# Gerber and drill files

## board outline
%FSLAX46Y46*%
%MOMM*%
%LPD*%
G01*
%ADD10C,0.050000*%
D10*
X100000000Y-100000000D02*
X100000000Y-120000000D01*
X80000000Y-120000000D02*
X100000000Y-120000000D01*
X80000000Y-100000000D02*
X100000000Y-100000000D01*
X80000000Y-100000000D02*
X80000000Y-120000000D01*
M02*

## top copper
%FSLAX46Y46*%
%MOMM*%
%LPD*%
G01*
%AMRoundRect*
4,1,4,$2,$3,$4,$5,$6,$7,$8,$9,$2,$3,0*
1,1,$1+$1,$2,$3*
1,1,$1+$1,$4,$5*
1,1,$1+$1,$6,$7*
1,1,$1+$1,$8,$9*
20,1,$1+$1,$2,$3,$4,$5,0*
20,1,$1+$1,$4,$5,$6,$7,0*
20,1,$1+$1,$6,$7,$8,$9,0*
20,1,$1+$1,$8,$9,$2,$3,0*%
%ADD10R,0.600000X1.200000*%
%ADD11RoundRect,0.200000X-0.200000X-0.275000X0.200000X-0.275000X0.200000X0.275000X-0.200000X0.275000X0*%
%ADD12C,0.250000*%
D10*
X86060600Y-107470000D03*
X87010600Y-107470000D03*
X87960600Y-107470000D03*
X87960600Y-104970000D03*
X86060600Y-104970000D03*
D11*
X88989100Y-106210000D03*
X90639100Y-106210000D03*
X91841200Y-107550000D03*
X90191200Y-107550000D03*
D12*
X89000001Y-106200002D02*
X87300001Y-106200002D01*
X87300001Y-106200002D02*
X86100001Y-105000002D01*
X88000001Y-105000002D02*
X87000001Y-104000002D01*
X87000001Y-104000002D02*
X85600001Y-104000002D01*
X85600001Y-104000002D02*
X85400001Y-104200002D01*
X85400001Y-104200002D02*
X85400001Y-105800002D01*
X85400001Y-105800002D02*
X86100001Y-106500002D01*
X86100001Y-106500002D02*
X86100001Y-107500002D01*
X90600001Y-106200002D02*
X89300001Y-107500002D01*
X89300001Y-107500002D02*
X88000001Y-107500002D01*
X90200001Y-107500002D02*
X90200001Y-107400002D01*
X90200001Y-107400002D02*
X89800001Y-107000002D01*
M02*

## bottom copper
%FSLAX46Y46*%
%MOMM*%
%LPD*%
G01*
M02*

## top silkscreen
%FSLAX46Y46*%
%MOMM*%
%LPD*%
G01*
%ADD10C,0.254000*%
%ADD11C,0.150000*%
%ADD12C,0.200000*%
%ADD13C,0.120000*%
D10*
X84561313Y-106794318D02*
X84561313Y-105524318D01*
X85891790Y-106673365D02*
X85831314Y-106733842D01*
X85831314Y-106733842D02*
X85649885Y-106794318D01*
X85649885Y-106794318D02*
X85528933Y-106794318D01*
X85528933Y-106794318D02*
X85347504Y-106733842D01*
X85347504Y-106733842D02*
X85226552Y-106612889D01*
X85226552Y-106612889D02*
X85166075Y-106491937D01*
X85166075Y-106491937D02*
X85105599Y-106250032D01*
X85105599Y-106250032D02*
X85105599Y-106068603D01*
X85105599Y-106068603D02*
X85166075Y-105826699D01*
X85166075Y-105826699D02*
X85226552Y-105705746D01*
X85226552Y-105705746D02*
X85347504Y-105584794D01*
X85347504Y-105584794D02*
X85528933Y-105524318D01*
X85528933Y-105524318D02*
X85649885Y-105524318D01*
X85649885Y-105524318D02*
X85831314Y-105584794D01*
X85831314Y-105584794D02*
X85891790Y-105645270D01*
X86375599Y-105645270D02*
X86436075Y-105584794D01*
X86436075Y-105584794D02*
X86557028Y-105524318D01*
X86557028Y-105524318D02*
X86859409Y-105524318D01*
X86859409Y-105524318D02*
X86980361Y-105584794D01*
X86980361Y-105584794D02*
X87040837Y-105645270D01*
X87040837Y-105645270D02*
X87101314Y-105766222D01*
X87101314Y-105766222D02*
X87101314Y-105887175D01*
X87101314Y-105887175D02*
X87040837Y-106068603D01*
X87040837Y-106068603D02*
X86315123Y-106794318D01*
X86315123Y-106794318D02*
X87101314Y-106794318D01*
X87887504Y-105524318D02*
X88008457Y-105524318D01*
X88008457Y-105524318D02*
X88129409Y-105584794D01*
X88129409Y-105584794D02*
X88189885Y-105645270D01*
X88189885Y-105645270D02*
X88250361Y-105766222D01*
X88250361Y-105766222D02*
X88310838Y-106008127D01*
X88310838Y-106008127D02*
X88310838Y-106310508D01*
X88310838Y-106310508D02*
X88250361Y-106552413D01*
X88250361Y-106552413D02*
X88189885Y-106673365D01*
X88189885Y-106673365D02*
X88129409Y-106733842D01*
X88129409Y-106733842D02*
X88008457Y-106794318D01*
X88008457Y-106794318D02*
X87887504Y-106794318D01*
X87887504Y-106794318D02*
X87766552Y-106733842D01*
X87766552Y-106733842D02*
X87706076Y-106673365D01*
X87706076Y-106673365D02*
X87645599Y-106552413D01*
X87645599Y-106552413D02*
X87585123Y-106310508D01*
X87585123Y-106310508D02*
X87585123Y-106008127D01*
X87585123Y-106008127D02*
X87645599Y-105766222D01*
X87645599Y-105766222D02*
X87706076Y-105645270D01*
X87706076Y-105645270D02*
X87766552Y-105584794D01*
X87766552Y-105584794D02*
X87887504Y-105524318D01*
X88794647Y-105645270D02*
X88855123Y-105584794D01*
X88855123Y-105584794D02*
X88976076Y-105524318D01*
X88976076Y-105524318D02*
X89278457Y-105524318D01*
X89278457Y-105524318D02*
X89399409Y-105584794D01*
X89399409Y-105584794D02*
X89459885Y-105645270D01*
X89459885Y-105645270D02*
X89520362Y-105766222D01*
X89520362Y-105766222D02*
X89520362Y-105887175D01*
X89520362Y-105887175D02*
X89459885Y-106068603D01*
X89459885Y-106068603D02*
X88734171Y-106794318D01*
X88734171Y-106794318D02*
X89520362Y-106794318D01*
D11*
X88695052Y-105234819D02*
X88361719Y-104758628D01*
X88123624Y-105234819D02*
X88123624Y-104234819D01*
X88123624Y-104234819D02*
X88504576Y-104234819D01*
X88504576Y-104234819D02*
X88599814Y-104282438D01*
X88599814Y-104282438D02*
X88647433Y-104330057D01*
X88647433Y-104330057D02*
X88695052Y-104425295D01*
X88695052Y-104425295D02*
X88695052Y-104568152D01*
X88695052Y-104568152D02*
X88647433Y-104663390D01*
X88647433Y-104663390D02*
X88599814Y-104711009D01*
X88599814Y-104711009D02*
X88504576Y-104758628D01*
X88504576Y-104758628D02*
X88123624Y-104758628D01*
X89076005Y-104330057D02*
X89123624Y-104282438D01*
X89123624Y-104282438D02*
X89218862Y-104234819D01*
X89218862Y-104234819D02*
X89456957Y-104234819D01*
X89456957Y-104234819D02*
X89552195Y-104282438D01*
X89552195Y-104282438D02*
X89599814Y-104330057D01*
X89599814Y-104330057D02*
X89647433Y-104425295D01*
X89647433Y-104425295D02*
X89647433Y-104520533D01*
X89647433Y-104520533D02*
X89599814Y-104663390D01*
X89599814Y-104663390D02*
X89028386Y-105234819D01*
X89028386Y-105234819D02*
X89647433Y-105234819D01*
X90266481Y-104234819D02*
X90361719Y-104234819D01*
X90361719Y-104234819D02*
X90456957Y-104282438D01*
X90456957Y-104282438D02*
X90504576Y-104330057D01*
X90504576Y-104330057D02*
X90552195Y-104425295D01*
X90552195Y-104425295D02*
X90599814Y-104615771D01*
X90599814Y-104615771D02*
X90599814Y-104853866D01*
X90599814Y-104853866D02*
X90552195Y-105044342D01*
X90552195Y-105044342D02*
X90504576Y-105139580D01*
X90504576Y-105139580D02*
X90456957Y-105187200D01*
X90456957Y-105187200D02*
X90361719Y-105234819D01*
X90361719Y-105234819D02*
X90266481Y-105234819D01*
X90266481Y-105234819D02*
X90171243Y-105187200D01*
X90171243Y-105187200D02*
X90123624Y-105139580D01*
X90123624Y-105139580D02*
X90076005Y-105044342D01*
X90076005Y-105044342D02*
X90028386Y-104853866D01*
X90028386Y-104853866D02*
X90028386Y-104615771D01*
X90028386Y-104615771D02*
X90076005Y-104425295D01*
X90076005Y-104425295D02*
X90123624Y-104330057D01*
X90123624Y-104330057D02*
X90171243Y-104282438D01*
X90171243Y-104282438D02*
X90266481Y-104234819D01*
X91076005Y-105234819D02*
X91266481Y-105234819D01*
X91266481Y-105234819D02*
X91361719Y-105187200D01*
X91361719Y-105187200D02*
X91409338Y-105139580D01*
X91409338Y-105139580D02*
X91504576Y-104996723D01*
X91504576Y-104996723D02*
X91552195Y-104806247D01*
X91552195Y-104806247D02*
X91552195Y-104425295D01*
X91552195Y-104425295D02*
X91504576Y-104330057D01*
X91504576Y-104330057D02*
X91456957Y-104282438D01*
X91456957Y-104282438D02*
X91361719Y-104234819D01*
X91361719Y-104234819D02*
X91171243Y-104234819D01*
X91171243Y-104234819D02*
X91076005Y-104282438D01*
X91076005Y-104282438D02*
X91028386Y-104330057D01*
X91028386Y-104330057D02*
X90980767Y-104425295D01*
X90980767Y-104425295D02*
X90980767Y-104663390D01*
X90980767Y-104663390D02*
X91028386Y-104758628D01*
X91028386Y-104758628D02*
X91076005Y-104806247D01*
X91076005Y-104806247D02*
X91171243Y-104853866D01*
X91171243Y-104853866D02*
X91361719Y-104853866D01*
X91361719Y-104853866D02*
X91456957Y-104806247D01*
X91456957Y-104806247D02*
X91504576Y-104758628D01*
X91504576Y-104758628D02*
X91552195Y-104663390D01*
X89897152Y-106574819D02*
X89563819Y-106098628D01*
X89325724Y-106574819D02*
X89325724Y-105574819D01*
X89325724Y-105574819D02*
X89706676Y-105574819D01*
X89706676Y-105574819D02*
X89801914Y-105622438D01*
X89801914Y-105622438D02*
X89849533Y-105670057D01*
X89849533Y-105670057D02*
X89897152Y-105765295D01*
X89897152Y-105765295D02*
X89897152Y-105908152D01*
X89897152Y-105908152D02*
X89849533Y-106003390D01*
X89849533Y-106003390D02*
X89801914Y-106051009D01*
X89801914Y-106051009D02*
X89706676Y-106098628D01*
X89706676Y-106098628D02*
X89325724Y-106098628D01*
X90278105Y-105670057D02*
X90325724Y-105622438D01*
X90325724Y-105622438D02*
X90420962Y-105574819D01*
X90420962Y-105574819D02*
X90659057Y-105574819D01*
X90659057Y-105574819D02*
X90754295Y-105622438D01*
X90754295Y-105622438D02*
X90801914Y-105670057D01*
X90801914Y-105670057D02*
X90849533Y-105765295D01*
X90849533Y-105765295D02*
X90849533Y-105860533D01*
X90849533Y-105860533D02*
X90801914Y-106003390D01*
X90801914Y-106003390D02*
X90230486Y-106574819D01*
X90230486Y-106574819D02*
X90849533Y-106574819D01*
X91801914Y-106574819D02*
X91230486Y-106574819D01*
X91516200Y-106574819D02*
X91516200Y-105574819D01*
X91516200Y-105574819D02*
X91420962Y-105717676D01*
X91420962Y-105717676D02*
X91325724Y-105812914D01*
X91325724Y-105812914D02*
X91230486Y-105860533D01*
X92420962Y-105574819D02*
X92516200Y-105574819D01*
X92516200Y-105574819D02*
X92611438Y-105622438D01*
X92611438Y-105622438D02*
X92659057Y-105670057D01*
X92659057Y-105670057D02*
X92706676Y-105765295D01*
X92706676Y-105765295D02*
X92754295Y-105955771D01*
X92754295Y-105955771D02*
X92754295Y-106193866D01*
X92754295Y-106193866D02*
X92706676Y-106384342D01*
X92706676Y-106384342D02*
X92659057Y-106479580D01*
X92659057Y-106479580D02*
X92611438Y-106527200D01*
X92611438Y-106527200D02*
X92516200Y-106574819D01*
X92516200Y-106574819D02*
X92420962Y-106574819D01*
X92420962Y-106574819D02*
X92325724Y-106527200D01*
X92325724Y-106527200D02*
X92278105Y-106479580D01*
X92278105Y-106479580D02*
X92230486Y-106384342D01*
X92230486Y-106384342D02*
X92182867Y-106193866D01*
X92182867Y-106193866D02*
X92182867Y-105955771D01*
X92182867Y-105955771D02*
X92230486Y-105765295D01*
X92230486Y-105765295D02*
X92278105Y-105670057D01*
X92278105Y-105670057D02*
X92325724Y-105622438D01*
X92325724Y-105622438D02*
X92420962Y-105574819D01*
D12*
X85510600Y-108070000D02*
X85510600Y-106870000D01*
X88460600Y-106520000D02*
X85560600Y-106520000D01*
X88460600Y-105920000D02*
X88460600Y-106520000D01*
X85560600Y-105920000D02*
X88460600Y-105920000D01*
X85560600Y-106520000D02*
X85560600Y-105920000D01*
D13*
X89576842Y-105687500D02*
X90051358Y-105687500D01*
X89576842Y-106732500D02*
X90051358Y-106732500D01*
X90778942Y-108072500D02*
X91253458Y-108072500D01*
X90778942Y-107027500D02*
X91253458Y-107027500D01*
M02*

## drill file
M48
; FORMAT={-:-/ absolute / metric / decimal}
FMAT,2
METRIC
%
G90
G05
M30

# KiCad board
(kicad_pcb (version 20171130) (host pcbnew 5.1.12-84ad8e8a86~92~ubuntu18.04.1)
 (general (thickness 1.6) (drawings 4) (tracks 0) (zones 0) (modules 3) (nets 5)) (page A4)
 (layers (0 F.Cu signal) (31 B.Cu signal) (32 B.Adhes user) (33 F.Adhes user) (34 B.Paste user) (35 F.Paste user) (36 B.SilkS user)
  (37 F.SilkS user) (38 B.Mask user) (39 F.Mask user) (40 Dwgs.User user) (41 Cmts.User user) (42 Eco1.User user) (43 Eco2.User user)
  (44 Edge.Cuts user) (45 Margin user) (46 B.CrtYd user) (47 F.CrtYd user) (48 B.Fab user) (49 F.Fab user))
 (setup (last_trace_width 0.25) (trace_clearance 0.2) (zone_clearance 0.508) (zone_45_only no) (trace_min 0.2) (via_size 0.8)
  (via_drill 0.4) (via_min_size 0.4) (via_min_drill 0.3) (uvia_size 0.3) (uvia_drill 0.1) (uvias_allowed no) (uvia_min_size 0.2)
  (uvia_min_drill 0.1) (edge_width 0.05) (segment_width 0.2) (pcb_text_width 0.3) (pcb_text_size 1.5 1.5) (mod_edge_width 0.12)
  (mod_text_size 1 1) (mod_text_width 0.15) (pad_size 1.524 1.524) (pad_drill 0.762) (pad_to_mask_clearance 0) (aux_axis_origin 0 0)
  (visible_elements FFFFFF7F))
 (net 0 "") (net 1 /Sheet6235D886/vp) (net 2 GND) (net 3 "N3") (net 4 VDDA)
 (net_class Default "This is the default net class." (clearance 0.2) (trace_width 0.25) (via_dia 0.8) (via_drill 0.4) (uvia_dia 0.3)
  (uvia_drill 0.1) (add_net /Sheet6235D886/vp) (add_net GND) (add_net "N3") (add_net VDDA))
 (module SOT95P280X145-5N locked (layer F.Cu) (at 87.010600 106.220000 90.000000)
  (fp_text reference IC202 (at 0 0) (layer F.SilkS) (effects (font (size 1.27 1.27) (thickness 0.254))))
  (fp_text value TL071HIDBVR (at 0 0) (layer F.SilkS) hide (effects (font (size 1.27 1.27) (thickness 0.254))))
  (fp_line (start -1.85 -1.5) (end -0.65 -1.5) (layer F.SilkS) (width 0.2))
  (fp_line (start -0.3 1.45) (end -0.3 -1.45) (layer F.SilkS) (width 0.2))
  (fp_line (start 0.3 1.45) (end -0.3 1.45) (layer F.SilkS) (width 0.2))
  (fp_line (start 0.3 -1.45) (end 0.3 1.45) (layer F.SilkS) (width 0.2))
  (fp_line (start -0.3 -1.45) (end 0.3 -1.45) (layer F.SilkS) (width 0.2))
  (pad 1 smd rect (at -1.25 -0.95 180.000000) (size 0.6 1.2) (layers F.Cu F.Mask F.Paste) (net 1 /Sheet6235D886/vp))
  (pad 2 smd rect (at -1.25 0 180.000000) (size 0.6 1.2) (layers F.Cu F.Mask F.Paste) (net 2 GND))
  (pad 3 smd rect (at -1.25 0.95 180.000000) (size 0.6 1.2) (layers F.Cu F.Mask F.Paste) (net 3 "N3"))
  (pad 4 smd rect (at 1.25 0.95 180.000000) (size 0.6 1.2) (layers F.Cu F.Mask F.Paste) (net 1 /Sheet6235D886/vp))
  (pad 5 smd rect (at 1.25 -0.95 180.000000) (size 0.6 1.2) (layers F.Cu F.Mask F.Paste) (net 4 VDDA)))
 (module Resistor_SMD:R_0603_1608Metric (layer F.Cu) (at 89.814100 106.210000)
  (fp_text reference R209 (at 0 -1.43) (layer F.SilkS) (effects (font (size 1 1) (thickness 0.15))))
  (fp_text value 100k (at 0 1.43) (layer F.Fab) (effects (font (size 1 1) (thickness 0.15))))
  (fp_line (start -0.237258 -0.5225) (end 0.237258 -0.5225) (layer F.SilkS) (width 0.12))
  (fp_line (start -0.237258 0.5225) (end 0.237258 0.5225) (layer F.SilkS) (width 0.12))
  (pad 1 smd roundrect (at -0.825 0) (size 0.8 0.95) (layers F.Cu F.Mask F.Paste) (roundrect_rratio 0.25) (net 4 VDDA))
  (pad 2 smd roundrect (at 0.825 0) (size 0.8 0.95) (layers F.Cu F.Mask F.Paste) (roundrect_rratio 0.25) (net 3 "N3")))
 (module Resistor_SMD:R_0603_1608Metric (layer F.Cu) (at 91.016200 107.550000)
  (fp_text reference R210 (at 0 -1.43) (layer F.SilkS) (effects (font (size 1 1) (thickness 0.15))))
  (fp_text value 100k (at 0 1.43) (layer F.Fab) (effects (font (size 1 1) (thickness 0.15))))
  (fp_line (start -0.237258 0.5225) (end 0.237258 0.5225) (layer F.SilkS) (width 0.12))
  (fp_line (start -0.237258 -0.5225) (end 0.237258 -0.5225) (layer F.SilkS) (width 0.12))
  (pad 2 smd roundrect (at 0.825 0) (size 0.8 0.95) (layers F.Cu F.Mask F.Paste) (roundrect_rratio 0.25) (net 2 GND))
  (pad 1 smd roundrect (at -0.825 0) (size 0.8 0.95) (layers F.Cu F.Mask F.Paste) (roundrect_rratio 0.25) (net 3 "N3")))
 (gr_line (start 100 100) (end 100 120) (layer Edge.Cuts) (width 0.05))
 (gr_line (start 80 120) (end 100 120) (layer Edge.Cuts) (width 0.05))
 (gr_line (start 80 100) (end 100 100) (layer Edge.Cuts) (width 0.05))
 (gr_line (start 80 100) (end 80 120) (layer Edge.Cuts) (width 0.05))
 (segment (start 89.000001 106.200002) (end 87.300001 106.200002) (width 0.250000) (layer F.Cu) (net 4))
 (segment (start 87.300001 106.200002) (end 86.100001 105.000002) (width 0.250000) (layer F.Cu) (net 4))
 (segment (start 88.000001 105.000002) (end 87.000001 104.000002) (width 0.250000) (layer F.Cu) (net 1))
 (segment (start 87.000001 104.000002) (end 85.600001 104.000002) (width 0.250000) (layer F.Cu) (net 1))
 (segment (start 85.600001 104.000002) (end 85.400001 104.200002) (width 0.250000) (layer F.Cu) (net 1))
 (segment (start 85.400001 104.200002) (end 85.400001 105.800002) (width 0.250000) (layer F.Cu) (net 1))
 (segment (start 85.400001 105.800002) (end 86.100001 106.500002) (width 0.250000) (layer F.Cu) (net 1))
 (segment (start 86.100001 106.500002) (end 86.100001 107.500002) (width 0.250000) (layer F.Cu) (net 1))
 (segment (start 90.600001 106.200002) (end 89.300001 107.500002) (width 0.250000) (layer F.Cu) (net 3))
 (segment (start 89.300001 107.500002) (end 88.000001 107.500002) (width 0.250000) (layer F.Cu) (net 3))
 (segment (start 90.200001 107.500002) (end 90.200001 107.400002) (width 0.250000) (layer F.Cu) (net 3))
 (segment (start 90.200001 107.400002) (end 89.800001 107.000002) (width 0.250000) (layer F.Cu) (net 3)))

